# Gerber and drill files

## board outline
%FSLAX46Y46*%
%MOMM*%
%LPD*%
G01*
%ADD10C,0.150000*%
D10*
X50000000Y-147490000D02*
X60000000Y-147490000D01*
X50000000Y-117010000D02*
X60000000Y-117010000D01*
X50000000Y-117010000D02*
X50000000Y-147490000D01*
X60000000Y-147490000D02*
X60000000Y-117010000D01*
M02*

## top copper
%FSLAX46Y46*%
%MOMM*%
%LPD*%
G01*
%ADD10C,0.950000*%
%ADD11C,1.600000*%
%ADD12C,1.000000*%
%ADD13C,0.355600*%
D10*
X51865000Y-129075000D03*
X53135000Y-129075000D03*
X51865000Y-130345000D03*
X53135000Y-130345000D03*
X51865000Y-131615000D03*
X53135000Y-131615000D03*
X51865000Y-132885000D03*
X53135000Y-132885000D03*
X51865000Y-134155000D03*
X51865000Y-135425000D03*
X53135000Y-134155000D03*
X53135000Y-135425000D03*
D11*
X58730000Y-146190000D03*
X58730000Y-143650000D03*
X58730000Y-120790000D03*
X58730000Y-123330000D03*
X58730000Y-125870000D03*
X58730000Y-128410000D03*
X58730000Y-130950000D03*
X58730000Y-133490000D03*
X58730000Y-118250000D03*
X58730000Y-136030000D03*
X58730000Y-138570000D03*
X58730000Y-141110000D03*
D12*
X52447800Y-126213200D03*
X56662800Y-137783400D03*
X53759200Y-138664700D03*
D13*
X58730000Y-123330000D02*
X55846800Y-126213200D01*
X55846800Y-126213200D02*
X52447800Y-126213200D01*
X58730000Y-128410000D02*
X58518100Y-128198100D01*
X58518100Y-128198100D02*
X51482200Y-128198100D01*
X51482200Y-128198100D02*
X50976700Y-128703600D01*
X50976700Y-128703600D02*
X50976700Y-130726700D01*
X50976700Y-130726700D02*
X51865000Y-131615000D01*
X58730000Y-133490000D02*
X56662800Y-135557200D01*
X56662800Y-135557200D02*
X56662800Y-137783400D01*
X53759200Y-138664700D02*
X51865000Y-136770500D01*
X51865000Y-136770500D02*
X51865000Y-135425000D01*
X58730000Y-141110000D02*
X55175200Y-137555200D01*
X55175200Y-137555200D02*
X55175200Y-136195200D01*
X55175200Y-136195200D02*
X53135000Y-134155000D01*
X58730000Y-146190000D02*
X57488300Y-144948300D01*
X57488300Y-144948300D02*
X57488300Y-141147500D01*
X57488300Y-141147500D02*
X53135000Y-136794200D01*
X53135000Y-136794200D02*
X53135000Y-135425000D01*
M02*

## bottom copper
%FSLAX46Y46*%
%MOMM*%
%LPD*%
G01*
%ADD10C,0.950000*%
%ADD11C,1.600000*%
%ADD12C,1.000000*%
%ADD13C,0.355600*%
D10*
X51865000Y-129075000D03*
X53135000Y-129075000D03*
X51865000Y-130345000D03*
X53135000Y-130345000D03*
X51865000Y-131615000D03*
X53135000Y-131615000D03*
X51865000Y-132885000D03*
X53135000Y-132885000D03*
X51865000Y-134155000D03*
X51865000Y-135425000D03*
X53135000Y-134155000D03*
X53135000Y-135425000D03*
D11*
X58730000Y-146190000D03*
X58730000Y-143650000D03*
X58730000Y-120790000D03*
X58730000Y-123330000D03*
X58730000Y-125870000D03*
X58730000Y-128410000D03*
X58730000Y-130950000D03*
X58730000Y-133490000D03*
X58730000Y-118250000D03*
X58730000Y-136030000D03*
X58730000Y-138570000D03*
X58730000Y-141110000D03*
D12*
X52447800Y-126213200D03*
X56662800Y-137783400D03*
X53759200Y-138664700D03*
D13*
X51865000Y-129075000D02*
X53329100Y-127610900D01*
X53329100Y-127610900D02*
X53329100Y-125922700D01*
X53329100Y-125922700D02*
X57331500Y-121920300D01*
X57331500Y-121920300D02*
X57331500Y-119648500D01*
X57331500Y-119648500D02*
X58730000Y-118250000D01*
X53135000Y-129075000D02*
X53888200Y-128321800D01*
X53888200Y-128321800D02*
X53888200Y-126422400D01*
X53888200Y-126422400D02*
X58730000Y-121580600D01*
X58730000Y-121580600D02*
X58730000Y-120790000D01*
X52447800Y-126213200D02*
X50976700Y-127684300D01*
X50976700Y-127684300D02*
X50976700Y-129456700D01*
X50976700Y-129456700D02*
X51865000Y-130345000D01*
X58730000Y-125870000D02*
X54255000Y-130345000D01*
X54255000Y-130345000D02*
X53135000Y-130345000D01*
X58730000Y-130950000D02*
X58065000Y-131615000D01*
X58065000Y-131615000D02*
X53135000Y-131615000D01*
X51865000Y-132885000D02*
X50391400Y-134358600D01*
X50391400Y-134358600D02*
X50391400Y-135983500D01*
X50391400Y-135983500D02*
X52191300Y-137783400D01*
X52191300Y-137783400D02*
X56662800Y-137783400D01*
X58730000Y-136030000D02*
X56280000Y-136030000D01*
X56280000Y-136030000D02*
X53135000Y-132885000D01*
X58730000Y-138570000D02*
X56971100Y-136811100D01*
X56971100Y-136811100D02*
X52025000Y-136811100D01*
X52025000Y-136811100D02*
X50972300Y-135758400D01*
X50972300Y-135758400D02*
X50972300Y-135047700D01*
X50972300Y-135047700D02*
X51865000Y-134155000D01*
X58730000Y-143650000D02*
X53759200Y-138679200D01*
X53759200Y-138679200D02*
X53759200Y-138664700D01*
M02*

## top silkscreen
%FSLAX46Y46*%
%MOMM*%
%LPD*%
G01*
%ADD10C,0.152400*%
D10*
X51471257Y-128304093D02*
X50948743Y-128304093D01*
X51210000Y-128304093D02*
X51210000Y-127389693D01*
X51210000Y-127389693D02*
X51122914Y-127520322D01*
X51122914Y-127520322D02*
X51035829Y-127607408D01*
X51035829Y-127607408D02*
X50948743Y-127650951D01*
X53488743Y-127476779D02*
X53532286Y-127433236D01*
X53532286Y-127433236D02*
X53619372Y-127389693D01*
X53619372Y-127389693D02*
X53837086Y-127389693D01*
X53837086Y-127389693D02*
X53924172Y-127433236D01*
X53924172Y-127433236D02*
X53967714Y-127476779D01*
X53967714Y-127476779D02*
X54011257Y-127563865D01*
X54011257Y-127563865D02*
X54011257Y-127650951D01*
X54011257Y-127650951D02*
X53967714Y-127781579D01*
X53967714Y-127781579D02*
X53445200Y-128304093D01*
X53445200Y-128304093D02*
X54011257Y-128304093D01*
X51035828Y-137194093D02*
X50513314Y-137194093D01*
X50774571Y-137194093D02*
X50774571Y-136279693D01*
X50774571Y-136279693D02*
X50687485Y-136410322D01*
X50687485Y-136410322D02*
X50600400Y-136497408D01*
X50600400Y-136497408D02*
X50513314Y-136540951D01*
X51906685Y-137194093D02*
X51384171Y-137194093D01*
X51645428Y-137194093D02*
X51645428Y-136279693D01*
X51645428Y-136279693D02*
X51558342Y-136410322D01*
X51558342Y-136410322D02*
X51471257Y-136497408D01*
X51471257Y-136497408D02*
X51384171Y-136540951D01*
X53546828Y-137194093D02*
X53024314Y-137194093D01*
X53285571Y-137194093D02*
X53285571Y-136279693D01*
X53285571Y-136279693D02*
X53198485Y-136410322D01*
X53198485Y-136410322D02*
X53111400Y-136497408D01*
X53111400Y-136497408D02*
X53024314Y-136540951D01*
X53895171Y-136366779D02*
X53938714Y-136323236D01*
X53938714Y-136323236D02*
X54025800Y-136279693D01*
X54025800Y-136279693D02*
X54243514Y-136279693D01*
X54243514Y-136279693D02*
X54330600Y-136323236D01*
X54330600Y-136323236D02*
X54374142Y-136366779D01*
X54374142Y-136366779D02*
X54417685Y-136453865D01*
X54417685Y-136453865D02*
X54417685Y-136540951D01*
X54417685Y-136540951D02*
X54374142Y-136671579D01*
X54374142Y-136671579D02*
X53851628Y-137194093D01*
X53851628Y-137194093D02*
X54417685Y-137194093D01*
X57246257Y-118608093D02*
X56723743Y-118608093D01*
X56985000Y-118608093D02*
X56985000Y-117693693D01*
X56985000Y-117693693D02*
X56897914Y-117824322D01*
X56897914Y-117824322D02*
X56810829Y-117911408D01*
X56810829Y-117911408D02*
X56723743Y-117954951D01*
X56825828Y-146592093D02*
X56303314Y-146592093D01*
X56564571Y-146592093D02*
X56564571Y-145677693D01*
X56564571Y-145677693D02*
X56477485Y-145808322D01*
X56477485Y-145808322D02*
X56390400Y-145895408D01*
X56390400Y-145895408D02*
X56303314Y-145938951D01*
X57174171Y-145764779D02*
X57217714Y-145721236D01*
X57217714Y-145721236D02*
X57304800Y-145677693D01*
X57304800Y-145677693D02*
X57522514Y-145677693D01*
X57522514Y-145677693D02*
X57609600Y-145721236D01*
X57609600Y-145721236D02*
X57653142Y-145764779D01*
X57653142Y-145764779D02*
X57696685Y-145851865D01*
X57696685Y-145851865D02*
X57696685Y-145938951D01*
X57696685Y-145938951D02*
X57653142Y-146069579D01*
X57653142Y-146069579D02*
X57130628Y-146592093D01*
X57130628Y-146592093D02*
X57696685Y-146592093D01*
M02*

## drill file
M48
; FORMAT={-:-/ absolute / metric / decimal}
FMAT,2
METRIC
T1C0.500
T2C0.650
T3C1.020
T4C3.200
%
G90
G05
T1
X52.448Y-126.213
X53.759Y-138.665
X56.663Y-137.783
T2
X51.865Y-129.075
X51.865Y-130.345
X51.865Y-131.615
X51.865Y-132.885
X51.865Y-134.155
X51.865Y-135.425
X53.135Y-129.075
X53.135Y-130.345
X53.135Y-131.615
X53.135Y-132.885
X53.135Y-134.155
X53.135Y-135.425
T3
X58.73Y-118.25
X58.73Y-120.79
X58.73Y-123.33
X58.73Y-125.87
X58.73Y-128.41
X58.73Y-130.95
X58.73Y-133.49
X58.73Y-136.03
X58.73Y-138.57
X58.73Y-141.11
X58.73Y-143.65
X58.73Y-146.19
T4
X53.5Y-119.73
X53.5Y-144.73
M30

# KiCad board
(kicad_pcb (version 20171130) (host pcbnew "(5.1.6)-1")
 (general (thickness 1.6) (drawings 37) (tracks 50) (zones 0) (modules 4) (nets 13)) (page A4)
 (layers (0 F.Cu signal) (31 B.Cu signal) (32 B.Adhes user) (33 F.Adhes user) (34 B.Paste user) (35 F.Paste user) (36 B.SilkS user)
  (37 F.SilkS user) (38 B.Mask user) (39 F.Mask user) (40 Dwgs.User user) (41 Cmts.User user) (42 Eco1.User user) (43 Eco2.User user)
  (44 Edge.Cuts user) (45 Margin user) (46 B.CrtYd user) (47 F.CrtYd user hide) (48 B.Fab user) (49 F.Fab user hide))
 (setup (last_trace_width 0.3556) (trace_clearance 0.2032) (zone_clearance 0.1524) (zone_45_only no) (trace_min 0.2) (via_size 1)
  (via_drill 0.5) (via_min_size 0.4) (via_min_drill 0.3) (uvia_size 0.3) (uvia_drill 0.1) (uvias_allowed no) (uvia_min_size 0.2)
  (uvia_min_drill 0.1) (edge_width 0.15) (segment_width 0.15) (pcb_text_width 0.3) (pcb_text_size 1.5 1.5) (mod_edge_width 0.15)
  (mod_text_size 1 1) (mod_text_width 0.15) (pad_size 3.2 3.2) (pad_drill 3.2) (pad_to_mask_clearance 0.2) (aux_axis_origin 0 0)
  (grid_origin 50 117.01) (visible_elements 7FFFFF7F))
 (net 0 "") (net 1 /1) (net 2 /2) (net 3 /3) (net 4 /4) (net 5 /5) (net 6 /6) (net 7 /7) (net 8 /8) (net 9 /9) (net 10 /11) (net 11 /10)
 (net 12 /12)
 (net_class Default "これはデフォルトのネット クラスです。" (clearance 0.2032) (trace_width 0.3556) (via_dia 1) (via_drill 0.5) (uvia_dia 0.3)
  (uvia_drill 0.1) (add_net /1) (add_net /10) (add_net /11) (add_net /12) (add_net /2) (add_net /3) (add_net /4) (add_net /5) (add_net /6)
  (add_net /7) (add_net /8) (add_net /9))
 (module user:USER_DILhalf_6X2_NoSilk (layer F.Cu) (at 52.5 132.25)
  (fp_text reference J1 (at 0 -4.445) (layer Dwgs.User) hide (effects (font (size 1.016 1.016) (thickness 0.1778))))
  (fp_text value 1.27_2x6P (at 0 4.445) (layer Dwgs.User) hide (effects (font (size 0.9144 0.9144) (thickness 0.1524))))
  (pad 1 thru_hole circle (at -0.635 -3.175) (size 0.95 0.95) (drill 0.65) (layers *.Cu *.Mask) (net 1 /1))
  (pad 2 thru_hole circle (at 0.635 -3.175) (size 0.95 0.95) (drill 0.65) (layers *.Cu *.Mask) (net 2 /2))
  (pad 3 thru_hole circle (at -0.635 -1.905) (size 0.95 0.95) (drill 0.65) (layers *.Cu *.Mask) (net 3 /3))
  (pad 4 thru_hole circle (at 0.635 -1.905) (size 0.95 0.95) (drill 0.65) (layers *.Cu *.Mask) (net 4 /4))
  (pad 5 thru_hole circle (at -0.635 -0.635) (size 0.95 0.95) (drill 0.65) (layers *.Cu *.Mask) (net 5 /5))
  (pad 6 thru_hole circle (at 0.635 -0.635) (size 0.95 0.95) (drill 0.65) (layers *.Cu *.Mask) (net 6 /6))
  (pad 7 thru_hole circle (at -0.635 0.635) (size 0.95 0.95) (drill 0.65) (layers *.Cu *.Mask) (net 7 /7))
  (pad 8 thru_hole circle (at 0.635 0.635) (size 0.95 0.95) (drill 0.65) (layers *.Cu *.Mask) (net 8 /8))
  (pad 9 thru_hole circle (at -0.635 1.905) (size 0.95 0.95) (drill 0.65) (layers *.Cu *.Mask) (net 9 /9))
  (pad 11 thru_hole circle (at -0.635 3.175) (size 0.95 0.95) (drill 0.65) (layers *.Cu *.Mask) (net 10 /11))
  (pad 10 thru_hole circle (at 0.635 1.905) (size 0.95 0.95) (drill 0.65) (layers *.Cu *.Mask) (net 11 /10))
  (pad 12 thru_hole circle (at 0.635 3.175) (size 0.95 0.95) (drill 0.65) (layers *.Cu *.Mask) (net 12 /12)))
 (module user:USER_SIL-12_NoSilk (layer F.Cu) (at 58.73 132.22 270)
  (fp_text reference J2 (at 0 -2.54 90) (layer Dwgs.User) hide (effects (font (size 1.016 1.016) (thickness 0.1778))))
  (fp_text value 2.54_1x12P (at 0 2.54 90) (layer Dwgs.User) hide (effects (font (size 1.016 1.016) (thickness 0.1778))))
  (pad 12 thru_hole circle (at 13.97 0 270) (size 1.6 1.6) (drill 1.02) (layers *.Cu *.Mask) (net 12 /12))
  (pad 11 thru_hole circle (at 11.43 0 270) (size 1.6 1.6) (drill 1.02) (layers *.Cu *.Mask) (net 10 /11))
  (pad 2 thru_hole circle (at -11.43 0 270) (size 1.6 1.6) (drill 1.02) (layers *.Cu *.Mask) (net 2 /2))
  (pad 3 thru_hole circle (at -8.89 0 270) (size 1.6 1.6) (drill 1.02) (layers *.Cu *.Mask) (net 3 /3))
  (pad 4 thru_hole circle (at -6.35 0 270) (size 1.6 1.6) (drill 1.02) (layers *.Cu *.Mask) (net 4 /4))
  (pad 5 thru_hole circle (at -3.81 0 270) (size 1.6 1.6) (drill 1.02) (layers *.Cu *.Mask) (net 5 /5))
  (pad 6 thru_hole circle (at -1.27 0 270) (size 1.6 1.6) (drill 1.02) (layers *.Cu *.Mask) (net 6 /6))
  (pad 7 thru_hole circle (at 1.27 0 270) (size 1.6 1.6) (drill 1.02) (layers *.Cu *.Mask) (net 7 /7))
  (pad 1 thru_hole circle (at -13.97 0 270) (size 1.6 1.6) (drill 1.02) (layers *.Cu *.Mask) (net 1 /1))
  (pad 8 thru_hole circle (at 3.81 0 270) (size 1.6 1.6) (drill 1.02) (layers *.Cu *.Mask) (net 8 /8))
  (pad 9 thru_hole circle (at 6.35 0 270) (size 1.6 1.6) (drill 1.02) (layers *.Cu *.Mask) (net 9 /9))
  (pad 10 thru_hole circle (at 8.89 0 270) (size 1.6 1.6) (drill 1.02) (layers *.Cu *.Mask) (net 11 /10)))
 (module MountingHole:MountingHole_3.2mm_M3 (layer F.Cu) (at 53.5 119.73)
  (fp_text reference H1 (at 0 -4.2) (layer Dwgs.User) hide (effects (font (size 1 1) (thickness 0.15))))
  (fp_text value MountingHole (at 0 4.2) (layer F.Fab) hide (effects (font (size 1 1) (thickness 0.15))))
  (pad 1 np_thru_hole circle (at 0 0) (size 3.2 3.2) (drill 3.2) (layers *.Cu *.Mask)))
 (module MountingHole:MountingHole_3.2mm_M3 (layer F.Cu) (at 53.5 144.73)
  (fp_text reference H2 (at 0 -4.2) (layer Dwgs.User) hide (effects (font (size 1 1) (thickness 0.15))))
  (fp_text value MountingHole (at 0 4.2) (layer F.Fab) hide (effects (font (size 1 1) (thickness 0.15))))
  (pad 1 np_thru_hole circle (at 0 0) (size 3.2 3.2) (drill 3.2) (layers *.Cu *.Mask)))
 (gr_line (start 50 147.49) (end 60 147.49) (angle 90) (layer Edge.Cuts) (width 0.15))
 (gr_line (start 50 117.01) (end 60 117.01) (angle 90) (layer Edge.Cuts) (width 0.15))
 (gr_line (start 50 117.01) (end 50 147.49) (angle 90) (layer Edge.Cuts) (width 0.15))
 (gr_line (start 60 147.49) (end 60 117.01) (angle 90) (layer Edge.Cuts) (width 0.15))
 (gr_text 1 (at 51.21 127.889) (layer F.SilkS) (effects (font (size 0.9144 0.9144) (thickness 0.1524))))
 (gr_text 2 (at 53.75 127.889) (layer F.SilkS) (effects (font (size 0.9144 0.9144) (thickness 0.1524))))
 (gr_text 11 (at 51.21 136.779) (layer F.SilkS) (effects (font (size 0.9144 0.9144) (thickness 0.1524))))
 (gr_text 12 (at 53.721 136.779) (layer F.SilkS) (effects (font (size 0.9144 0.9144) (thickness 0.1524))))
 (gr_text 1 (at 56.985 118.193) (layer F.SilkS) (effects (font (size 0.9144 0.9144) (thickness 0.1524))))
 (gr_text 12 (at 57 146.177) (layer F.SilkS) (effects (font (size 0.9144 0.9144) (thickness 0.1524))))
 (segment (start 51.865 129.075) (end 53.3291 127.6109) (width 0.3556) (layer B.Cu) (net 1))
 (segment (start 53.3291 127.6109) (end 53.3291 125.9227) (width 0.3556) (layer B.Cu) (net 1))
 (segment (start 53.3291 125.9227) (end 57.3315 121.9203) (width 0.3556) (layer B.Cu) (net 1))
 (segment (start 57.3315 121.9203) (end 57.3315 119.6485) (width 0.3556) (layer B.Cu) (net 1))
 (segment (start 57.3315 119.6485) (end 58.73 118.25) (width 0.3556) (layer B.Cu) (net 1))
 (segment (start 53.135 129.075) (end 53.8882 128.3218) (width 0.3556) (layer B.Cu) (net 2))
 (segment (start 53.8882 128.3218) (end 53.8882 126.4224) (width 0.3556) (layer B.Cu) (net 2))
 (segment (start 53.8882 126.4224) (end 58.73 121.5806) (width 0.3556) (layer B.Cu) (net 2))
 (segment (start 58.73 121.5806) (end 58.73 120.79) (width 0.3556) (layer B.Cu) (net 2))
 (segment (start 52.4478 126.2132) (end 50.9767 127.6843) (width 0.3556) (layer B.Cu) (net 3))
 (segment (start 50.9767 127.6843) (end 50.9767 129.4567) (width 0.3556) (layer B.Cu) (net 3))
 (segment (start 50.9767 129.4567) (end 51.865 130.345) (width 0.3556) (layer B.Cu) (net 3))
 (segment (start 58.73 123.33) (end 55.8468 126.2132) (width 0.3556) (layer F.Cu) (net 3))
 (segment (start 55.8468 126.2132) (end 52.4478 126.2132) (width 0.3556) (layer F.Cu) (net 3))
 (via (at 52.4478 126.2132) (size 1) (layers F.Cu B.Cu) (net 3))
 (segment (start 58.73 125.87) (end 54.255 130.345) (width 0.3556) (layer B.Cu) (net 4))
 (segment (start 54.255 130.345) (end 53.135 130.345) (width 0.3556) (layer B.Cu) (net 4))
 (segment (start 58.73 128.41) (end 58.5181 128.1981) (width 0.3556) (layer F.Cu) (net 5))
 (segment (start 58.5181 128.1981) (end 51.4822 128.1981) (width 0.3556) (layer F.Cu) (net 5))
 (segment (start 51.4822 128.1981) (end 50.9767 128.7036) (width 0.3556) (layer F.Cu) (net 5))
 (segment (start 50.9767 128.7036) (end 50.9767 130.7267) (width 0.3556) (layer F.Cu) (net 5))
 (segment (start 50.9767 130.7267) (end 51.865 131.615) (width 0.3556) (layer F.Cu) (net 5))
 (segment (start 58.73 130.95) (end 58.065 131.615) (width 0.3556) (layer B.Cu) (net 6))
 (segment (start 58.065 131.615) (end 53.135 131.615) (width 0.3556) (layer B.Cu) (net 6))
 (segment (start 58.73 133.49) (end 56.6628 135.5572) (width 0.3556) (layer F.Cu) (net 7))
 (segment (start 56.6628 135.5572) (end 56.6628 137.7834) (width 0.3556) (layer F.Cu) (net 7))
 (segment (start 51.865 132.885) (end 50.3914 134.3586) (width 0.3556) (layer B.Cu) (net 7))
 (segment (start 50.3914 134.3586) (end 50.3914 135.9835) (width 0.3556) (layer B.Cu) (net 7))
 (segment (start 50.3914 135.9835) (end 52.1913 137.7834) (width 0.3556) (layer B.Cu) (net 7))
 (segment (start 52.1913 137.7834) (end 56.6628 137.7834) (width 0.3556) (layer B.Cu) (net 7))
 (via (at 56.6628 137.7834) (size 1) (layers F.Cu B.Cu) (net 7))
 (segment (start 58.73 136.03) (end 56.28 136.03) (width 0.3556) (layer B.Cu) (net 8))
 (segment (start 56.28 136.03) (end 53.135 132.885) (width 0.3556) (layer B.Cu) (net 8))
 (segment (start 58.73 138.57) (end 56.9711 136.8111) (width 0.3556) (layer B.Cu) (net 9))
 (segment (start 56.9711 136.8111) (end 52.025 136.8111) (width 0.3556) (layer B.Cu) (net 9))
 (segment (start 52.025 136.8111) (end 50.9723 135.7584) (width 0.3556) (layer B.Cu) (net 9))
 (segment (start 50.9723 135.7584) (end 50.9723 135.0477) (width 0.3556) (layer B.Cu) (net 9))
 (segment (start 50.9723 135.0477) (end 51.865 134.155) (width 0.3556) (layer B.Cu) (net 9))
 (segment (start 53.7592 138.6647) (end 51.865 136.7705) (width 0.3556) (layer F.Cu) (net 10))
 (segment (start 51.865 136.7705) (end 51.865 135.425) (width 0.3556) (layer F.Cu) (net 10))
 (segment (start 58.73 143.65) (end 53.7592 138.6792) (width 0.3556) (layer B.Cu) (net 10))
 (segment (start 53.7592 138.6792) (end 53.7592 138.6647) (width 0.3556) (layer B.Cu) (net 10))
 (via (at 53.7592 138.6647) (size 1) (layers F.Cu B.Cu) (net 10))
 (segment (start 58.73 141.11) (end 55.1752 137.5552) (width 0.3556) (layer F.Cu) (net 11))
 (segment (start 55.1752 137.5552) (end 55.1752 136.1952) (width 0.3556) (layer F.Cu) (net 11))
 (segment (start 55.1752 136.1952) (end 53.135 134.155) (width 0.3556) (layer F.Cu) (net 11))
 (segment (start 58.73 146.19) (end 57.4883 144.9483) (width 0.3556) (layer F.Cu) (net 12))
 (segment (start 57.4883 144.9483) (end 57.4883 141.1475) (width 0.3556) (layer F.Cu) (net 12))
 (segment (start 57.4883 141.1475) (end 53.135 136.7942) (width 0.3556) (layer F.Cu) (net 12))
 (segment (start 53.135 136.7942) (end 53.135 135.425) (width 0.3556) (layer F.Cu) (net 12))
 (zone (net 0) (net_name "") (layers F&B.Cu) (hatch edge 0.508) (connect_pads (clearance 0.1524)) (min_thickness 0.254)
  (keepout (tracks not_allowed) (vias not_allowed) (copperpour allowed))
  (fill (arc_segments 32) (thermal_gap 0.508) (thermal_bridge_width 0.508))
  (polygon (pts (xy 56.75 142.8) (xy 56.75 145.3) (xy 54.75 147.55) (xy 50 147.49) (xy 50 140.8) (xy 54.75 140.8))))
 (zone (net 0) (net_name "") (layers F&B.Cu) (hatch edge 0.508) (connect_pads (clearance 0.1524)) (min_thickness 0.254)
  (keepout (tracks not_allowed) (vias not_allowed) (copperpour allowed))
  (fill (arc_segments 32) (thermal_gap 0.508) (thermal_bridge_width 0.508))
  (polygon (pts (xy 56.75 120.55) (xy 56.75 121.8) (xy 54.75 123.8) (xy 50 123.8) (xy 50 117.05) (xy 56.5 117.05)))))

